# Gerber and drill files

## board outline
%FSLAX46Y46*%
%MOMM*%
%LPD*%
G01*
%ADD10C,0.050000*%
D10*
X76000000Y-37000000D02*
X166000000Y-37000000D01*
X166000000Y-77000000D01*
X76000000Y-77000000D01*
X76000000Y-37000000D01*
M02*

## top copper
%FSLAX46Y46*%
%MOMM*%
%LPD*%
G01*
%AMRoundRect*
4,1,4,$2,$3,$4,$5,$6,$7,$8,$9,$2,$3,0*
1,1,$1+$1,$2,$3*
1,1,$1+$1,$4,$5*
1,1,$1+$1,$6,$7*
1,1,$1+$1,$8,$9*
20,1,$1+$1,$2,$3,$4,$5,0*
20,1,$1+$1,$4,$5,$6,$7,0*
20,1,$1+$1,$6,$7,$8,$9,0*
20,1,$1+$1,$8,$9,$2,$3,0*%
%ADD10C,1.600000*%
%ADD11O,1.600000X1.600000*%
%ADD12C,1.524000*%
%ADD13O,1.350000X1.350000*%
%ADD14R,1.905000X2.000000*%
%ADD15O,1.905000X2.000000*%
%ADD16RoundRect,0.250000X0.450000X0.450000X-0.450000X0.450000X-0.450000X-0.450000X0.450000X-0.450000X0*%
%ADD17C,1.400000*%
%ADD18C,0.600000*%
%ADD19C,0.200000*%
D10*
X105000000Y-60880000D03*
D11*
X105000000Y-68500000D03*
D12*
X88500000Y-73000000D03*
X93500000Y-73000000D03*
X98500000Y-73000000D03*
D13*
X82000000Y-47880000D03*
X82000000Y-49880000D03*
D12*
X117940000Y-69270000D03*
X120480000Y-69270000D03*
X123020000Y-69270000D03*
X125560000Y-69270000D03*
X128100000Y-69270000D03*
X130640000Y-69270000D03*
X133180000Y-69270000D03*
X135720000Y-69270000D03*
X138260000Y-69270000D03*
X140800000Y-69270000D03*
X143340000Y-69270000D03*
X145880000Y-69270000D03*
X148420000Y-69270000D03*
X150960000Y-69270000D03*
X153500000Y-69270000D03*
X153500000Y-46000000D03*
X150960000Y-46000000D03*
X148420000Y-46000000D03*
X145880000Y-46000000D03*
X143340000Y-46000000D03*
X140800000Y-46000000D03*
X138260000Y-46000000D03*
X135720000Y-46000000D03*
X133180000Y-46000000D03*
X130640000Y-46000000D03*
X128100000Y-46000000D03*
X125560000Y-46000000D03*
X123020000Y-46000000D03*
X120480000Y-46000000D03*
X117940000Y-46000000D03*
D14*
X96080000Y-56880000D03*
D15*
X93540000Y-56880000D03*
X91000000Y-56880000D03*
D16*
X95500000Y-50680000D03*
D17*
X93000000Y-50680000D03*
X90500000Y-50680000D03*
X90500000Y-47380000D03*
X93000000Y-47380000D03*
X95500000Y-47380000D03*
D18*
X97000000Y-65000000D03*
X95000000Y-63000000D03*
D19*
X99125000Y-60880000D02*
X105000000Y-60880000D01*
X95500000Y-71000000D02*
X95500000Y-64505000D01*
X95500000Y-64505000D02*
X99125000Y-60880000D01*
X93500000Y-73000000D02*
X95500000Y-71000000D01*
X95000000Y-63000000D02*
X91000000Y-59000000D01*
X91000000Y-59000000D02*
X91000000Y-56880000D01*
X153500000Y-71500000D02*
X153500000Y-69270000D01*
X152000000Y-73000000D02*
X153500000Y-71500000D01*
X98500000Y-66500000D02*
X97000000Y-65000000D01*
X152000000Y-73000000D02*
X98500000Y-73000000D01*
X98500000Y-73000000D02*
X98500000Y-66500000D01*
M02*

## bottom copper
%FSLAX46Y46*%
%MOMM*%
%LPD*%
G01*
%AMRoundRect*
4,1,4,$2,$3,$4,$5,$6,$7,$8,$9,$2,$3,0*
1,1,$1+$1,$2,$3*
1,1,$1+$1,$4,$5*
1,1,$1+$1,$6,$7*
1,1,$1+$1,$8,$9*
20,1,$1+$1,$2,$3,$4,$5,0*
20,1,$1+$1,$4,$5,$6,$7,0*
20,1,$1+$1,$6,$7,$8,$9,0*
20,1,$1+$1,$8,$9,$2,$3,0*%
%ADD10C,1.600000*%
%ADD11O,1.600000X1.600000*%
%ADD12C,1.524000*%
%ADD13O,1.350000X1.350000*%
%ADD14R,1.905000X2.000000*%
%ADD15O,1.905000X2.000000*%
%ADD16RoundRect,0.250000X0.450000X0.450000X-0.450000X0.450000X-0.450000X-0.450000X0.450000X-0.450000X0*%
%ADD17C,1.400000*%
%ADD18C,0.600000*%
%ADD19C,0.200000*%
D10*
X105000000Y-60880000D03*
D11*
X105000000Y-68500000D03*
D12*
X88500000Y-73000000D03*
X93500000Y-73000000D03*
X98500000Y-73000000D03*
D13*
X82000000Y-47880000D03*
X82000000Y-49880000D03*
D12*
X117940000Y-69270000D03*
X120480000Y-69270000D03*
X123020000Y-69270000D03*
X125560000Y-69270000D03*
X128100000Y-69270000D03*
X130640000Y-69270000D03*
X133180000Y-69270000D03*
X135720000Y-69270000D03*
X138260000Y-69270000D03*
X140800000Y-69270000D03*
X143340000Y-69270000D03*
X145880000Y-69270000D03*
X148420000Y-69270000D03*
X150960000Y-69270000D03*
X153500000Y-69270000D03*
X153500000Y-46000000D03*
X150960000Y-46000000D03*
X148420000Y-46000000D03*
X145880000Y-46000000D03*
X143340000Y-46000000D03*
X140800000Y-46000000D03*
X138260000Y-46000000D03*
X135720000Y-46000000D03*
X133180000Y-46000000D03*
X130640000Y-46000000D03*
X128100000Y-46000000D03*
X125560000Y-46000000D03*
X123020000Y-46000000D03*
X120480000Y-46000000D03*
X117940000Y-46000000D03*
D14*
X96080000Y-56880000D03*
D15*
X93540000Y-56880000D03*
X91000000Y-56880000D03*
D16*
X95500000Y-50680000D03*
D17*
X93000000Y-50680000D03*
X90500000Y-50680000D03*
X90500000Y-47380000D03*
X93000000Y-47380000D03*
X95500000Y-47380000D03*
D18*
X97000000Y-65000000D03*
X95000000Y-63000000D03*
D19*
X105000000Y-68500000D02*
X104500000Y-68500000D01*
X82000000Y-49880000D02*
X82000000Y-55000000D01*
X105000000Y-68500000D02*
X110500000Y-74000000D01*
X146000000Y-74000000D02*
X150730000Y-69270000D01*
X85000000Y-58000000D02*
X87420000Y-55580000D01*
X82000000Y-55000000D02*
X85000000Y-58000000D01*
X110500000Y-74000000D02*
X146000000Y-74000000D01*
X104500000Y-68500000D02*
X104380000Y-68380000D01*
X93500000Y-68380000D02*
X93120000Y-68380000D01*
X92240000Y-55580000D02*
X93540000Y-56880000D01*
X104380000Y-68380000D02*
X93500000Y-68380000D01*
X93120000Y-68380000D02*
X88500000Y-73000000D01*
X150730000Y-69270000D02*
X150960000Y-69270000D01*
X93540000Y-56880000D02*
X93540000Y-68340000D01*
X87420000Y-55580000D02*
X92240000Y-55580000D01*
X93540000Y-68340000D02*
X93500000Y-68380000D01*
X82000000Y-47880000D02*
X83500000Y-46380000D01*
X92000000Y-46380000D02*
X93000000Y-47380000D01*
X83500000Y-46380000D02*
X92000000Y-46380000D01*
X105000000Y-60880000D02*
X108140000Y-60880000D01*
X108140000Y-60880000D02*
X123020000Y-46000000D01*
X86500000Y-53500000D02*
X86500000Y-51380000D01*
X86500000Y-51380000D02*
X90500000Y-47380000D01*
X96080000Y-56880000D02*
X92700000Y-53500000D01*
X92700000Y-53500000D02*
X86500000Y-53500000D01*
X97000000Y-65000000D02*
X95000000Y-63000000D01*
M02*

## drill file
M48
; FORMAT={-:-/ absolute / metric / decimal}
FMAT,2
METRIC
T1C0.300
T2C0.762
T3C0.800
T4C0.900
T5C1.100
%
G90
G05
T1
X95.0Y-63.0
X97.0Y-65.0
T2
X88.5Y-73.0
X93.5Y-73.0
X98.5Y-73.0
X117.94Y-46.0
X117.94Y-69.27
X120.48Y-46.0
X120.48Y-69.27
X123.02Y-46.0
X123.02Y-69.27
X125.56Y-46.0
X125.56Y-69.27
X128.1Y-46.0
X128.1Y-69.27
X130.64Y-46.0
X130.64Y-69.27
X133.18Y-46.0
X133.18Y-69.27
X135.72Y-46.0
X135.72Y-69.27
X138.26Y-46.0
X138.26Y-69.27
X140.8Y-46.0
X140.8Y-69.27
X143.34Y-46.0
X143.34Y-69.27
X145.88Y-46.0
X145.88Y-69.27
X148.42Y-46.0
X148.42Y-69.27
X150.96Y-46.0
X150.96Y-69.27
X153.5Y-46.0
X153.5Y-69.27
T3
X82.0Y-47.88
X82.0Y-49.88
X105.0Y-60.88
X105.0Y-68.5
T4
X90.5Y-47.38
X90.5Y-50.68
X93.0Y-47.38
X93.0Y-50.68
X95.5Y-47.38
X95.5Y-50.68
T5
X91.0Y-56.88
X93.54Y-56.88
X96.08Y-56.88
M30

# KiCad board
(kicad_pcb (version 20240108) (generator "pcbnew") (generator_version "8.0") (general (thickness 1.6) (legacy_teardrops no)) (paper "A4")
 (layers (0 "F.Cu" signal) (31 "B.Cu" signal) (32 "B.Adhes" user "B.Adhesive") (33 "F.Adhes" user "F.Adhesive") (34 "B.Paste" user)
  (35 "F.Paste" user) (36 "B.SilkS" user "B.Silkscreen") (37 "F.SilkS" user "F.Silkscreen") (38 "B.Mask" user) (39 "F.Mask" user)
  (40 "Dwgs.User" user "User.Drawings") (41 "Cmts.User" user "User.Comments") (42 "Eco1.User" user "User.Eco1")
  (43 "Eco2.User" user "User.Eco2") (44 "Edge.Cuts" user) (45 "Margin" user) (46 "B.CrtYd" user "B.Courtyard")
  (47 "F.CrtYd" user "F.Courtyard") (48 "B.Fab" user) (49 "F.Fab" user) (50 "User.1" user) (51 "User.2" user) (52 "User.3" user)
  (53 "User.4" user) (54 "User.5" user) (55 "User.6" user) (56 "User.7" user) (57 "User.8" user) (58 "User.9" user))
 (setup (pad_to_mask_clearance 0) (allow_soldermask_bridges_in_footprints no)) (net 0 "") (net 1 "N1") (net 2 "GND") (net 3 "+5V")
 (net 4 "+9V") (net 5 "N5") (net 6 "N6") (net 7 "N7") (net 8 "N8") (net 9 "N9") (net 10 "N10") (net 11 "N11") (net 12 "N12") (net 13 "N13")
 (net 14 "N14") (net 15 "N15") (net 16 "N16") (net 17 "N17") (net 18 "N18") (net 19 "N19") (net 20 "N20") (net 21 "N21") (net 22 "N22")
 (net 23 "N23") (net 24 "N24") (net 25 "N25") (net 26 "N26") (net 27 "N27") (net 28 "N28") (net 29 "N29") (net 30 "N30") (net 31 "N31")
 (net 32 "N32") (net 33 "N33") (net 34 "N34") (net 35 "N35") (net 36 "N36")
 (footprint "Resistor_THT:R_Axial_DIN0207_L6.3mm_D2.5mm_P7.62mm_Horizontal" (layer "F.Cu") (at 105 60.88 -90)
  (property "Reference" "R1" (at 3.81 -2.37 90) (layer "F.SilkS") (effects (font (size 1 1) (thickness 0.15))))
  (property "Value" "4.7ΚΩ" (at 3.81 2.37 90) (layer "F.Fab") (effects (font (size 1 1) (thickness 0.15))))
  (pad "1" thru_hole circle (at 0 0 270) (size 1.6 1.6) (drill 0.8) (layers "*.Cu" "*.Mask") (remove_unused_layers no) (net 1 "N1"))
  (pad "2" thru_hole oval (at 7.62 0 270) (size 1.6 1.6) (drill 0.8) (layers "*.Cu" "*.Mask") (remove_unused_layers no) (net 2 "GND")))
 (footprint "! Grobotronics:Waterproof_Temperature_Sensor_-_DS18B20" (layer "F.Cu") (at 93 66.5)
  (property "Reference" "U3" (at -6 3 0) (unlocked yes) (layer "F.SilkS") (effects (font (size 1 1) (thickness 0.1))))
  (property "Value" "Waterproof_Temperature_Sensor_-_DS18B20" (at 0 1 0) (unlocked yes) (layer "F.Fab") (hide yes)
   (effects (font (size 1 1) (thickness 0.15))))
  (pad "1" thru_hole circle (at -4.5 6.5) (size 1.524 1.524) (drill 0.762) (layers "*.Cu" "*.Mask") (remove_unused_layers no) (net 2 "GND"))
  (pad "2" thru_hole circle (at 0.5 6.5) (size 1.524 1.524) (drill 0.762) (layers "*.Cu" "*.Mask") (remove_unused_layers no) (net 1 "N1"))
  (pad "3" thru_hole circle (at 5.5 6.5) (size 1.524 1.524) (drill 0.762) (layers "*.Cu" "*.Mask") (remove_unused_layers no) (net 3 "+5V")))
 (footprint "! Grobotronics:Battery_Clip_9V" (layer "F.Cu") (at 82 48.38)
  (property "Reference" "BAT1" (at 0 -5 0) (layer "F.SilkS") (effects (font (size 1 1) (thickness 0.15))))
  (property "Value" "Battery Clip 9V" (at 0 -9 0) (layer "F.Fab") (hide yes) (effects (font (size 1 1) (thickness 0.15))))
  (pad "+" thru_hole oval (at 0 -0.5) (size 1.35 1.35) (drill 0.8) (layers "*.Cu" "*.Mask") (remove_unused_layers no) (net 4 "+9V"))
  (pad "-" thru_hole oval (at 0 1.5) (size 1.35 1.35) (drill 0.8) (layers "*.Cu" "*.Mask") (remove_unused_layers no) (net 2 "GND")))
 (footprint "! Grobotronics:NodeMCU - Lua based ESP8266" (layer "F.Cu") (at 135.72 57.77 90)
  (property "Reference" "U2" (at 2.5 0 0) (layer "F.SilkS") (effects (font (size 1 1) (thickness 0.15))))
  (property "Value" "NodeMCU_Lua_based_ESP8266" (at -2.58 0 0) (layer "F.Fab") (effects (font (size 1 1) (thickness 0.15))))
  (pad "1" thru_hole circle (at -11.5 -17.78 90) (size 1.524 1.524) (drill 0.762) (layers "*.Cu" "*.Mask") (remove_unused_layers no)
   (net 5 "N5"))
  (pad "2" thru_hole circle (at -11.5 -15.24 90) (size 1.524 1.524) (drill 0.762) (layers "*.Cu" "*.Mask") (remove_unused_layers no)
   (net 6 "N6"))
  (pad "3" thru_hole circle (at -11.5 -12.7 90) (size 1.524 1.524) (drill 0.762) (layers "*.Cu" "*.Mask") (remove_unused_layers no)
   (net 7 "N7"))
  (pad "4" thru_hole circle (at -11.5 -10.16 90) (size 1.524 1.524) (drill 0.762) (layers "*.Cu" "*.Mask") (remove_unused_layers no)
   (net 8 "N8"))
  (pad "5" thru_hole circle (at -11.5 -7.62 90) (size 1.524 1.524) (drill 0.762) (layers "*.Cu" "*.Mask") (remove_unused_layers no)
   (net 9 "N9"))
  (pad "6" thru_hole circle (at -11.5 -5.08 90) (size 1.524 1.524) (drill 0.762) (layers "*.Cu" "*.Mask") (remove_unused_layers no)
   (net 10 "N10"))
  (pad "7" thru_hole circle (at -11.5 -2.54 90) (size 1.524 1.524) (drill 0.762) (layers "*.Cu" "*.Mask") (remove_unused_layers no)
   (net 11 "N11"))
  (pad "8" thru_hole circle (at -11.5 0 90) (size 1.524 1.524) (drill 0.762) (layers "*.Cu" "*.Mask") (remove_unused_layers no)
   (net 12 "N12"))
  (pad "9" thru_hole circle (at -11.5 2.54 90) (size 1.524 1.524) (drill 0.762) (layers "*.Cu" "*.Mask") (remove_unused_layers no)
   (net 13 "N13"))
  (pad "10" thru_hole circle (at -11.5 5.08 90) (size 1.524 1.524) (drill 0.762) (layers "*.Cu" "*.Mask") (remove_unused_layers no)
   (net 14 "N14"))
  (pad "11" thru_hole circle (at -11.5 7.62 90) (size 1.524 1.524) (drill 0.762) (layers "*.Cu" "*.Mask") (remove_unused_layers no)
   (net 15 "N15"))
  (pad "12" thru_hole circle (at -11.5 10.16 90) (size 1.524 1.524) (drill 0.762) (layers "*.Cu" "*.Mask") (remove_unused_layers no)
   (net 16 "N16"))
  (pad "13" thru_hole circle (at -11.5 12.7 90) (size 1.524 1.524) (drill 0.762) (layers "*.Cu" "*.Mask") (remove_unused_layers no)
   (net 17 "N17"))
  (pad "14" thru_hole circle (at -11.5 15.24 90) (size 1.524 1.524) (drill 0.762) (layers "*.Cu" "*.Mask") (remove_unused_layers no)
   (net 2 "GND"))
  (pad "15" thru_hole circle (at -11.5 17.78 90) (size 1.524 1.524) (drill 0.762) (layers "*.Cu" "*.Mask") (remove_unused_layers no)
   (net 3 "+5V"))
  (pad "16" thru_hole circle (at 11.77 17.78 90) (size 1.524 1.524) (drill 0.762) (layers "*.Cu" "*.Mask") (remove_unused_layers no)
   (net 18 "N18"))
  (pad "17" thru_hole circle (at 11.77 15.24 90) (size 1.524 1.524) (drill 0.762) (layers "*.Cu" "*.Mask") (remove_unused_layers no)
   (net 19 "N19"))
  (pad "18" thru_hole circle (at 11.77 12.7 90) (size 1.524 1.524) (drill 0.762) (layers "*.Cu" "*.Mask") (remove_unused_layers no)
   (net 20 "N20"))
  (pad "19" thru_hole circle (at 11.77 10.16 90) (size 1.524 1.524) (drill 0.762) (layers "*.Cu" "*.Mask") (remove_unused_layers no)
   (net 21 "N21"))
  (pad "20" thru_hole circle (at 11.77 7.62 90) (size 1.524 1.524) (drill 0.762) (layers "*.Cu" "*.Mask") (remove_unused_layers no)
   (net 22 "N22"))
  (pad "21" thru_hole circle (at 11.77 5.08 90) (size 1.524 1.524) (drill 0.762) (layers "*.Cu" "*.Mask") (remove_unused_layers no)
   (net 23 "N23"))
  (pad "22" thru_hole circle (at 11.77 2.54 90) (size 1.524 1.524) (drill 0.762) (layers "*.Cu" "*.Mask") (remove_unused_layers no)
   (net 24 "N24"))
  (pad "23" thru_hole circle (at 11.77 0 90) (size 1.524 1.524) (drill 0.762) (layers "*.Cu" "*.Mask") (remove_unused_layers no)
   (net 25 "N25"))
  (pad "24" thru_hole circle (at 11.77 -2.54 90) (size 1.524 1.524) (drill 0.762) (layers "*.Cu" "*.Mask") (remove_unused_layers no)
   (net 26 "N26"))
  (pad "25" thru_hole circle (at 11.77 -5.08 90) (size 1.524 1.524) (drill 0.762) (layers "*.Cu" "*.Mask") (remove_unused_layers no)
   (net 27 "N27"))
  (pad "26" thru_hole circle (at 11.77 -7.62 90) (size 1.524 1.524) (drill 0.762) (layers "*.Cu" "*.Mask") (remove_unused_layers no)
   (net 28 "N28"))
  (pad "27" thru_hole circle (at 11.77 -10.16 90) (size 1.524 1.524) (drill 0.762) (layers "*.Cu" "*.Mask") (remove_unused_layers no)
   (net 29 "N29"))
  (pad "28" thru_hole circle (at 11.77 -12.7 90) (size 1.524 1.524) (drill 0.762) (layers "*.Cu" "*.Mask") (remove_unused_layers no)
   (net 1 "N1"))
  (pad "29" thru_hole circle (at 11.77 -15.24 90) (size 1.524 1.524) (drill 0.762) (layers "*.Cu" "*.Mask") (remove_unused_layers no)
   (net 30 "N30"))
  (pad "30" thru_hole circle (at 11.77 -17.78 90) (size 1.524 1.524) (drill 0.762) (layers "*.Cu" "*.Mask") (remove_unused_layers no)
   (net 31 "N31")))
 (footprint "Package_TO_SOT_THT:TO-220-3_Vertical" (layer "F.Cu") (at 96.08 56.88 180)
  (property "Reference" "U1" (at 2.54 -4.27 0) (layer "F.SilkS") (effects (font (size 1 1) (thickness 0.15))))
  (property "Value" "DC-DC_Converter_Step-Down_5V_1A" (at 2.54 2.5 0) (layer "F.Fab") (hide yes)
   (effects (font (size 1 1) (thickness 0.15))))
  (pad "1" thru_hole rect (at 0 0 180) (size 1.905 2) (drill 1.1) (layers "*.Cu" "*.Mask") (remove_unused_layers no) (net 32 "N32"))
  (pad "2" thru_hole oval (at 2.54 0 180) (size 1.905 2) (drill 1.1) (layers "*.Cu" "*.Mask") (remove_unused_layers no) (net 2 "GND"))
  (pad "3" thru_hole oval (at 5.08 0 180) (size 1.905 2) (drill 1.1) (layers "*.Cu" "*.Mask") (remove_unused_layers no) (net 3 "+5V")))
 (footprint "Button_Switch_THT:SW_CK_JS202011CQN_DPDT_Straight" (layer "F.Cu") (at 95.5 50.68 180)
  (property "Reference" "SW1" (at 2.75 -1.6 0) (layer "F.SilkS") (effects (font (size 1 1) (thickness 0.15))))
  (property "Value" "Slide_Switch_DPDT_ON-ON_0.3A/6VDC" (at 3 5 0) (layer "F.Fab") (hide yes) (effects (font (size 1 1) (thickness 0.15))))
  (pad "1" thru_hole roundrect (at 0 0 180) (size 1.4 1.4) (drill 0.9) (layers "*.Cu" "*.Mask") (remove_unused_layers no)
   (roundrect_rratio 0.1785714286) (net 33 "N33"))
  (pad "2" thru_hole circle (at 2.5 0 180) (size 1.4 1.4) (drill 0.9) (layers "*.Cu" "*.Mask") (remove_unused_layers no) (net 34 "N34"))
  (pad "3" thru_hole circle (at 5 0 180) (size 1.4 1.4) (drill 0.9) (layers "*.Cu" "*.Mask") (remove_unused_layers no) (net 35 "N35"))
  (pad "4" thru_hole circle (at 5 3.3 180) (size 1.4 1.4) (drill 0.9) (layers "*.Cu" "*.Mask") (remove_unused_layers no) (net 32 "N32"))
  (pad "5" thru_hole circle (at 2.5 3.3 180) (size 1.4 1.4) (drill 0.9) (layers "*.Cu" "*.Mask") (remove_unused_layers no) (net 4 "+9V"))
  (pad "6" thru_hole circle (at 0 3.3 180) (size 1.4 1.4) (drill 0.9) (layers "*.Cu" "*.Mask") (remove_unused_layers no) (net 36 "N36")))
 (gr_rect (start 76 37) (end 166 77) (stroke (width 0.05) (type default)) (fill none) (layer "Edge.Cuts"))
 (segment (start 105 68.5) (end 104.5 68.5) (width 0.2) (layer "B.Cu") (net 2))
 (segment (start 82 49.88) (end 82 55) (width 0.2) (layer "B.Cu") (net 2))
 (segment (start 105 68.5) (end 110.5 74) (width 0.2) (layer "B.Cu") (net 2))
 (segment (start 146 74) (end 150.73 69.27) (width 0.2) (layer "B.Cu") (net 2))
 (segment (start 85 58) (end 87.42 55.58) (width 0.2) (layer "B.Cu") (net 2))
 (segment (start 82 55) (end 85 58) (width 0.2) (layer "B.Cu") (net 2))
 (segment (start 110.5 74) (end 146 74) (width 0.2) (layer "B.Cu") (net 2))
 (segment (start 104.5 68.5) (end 104.38 68.38) (width 0.2) (layer "B.Cu") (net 2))
 (segment (start 93.5 68.38) (end 93.12 68.38) (width 0.2) (layer "B.Cu") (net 2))
 (segment (start 92.24 55.58) (end 93.54 56.88) (width 0.2) (layer "B.Cu") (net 2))
 (segment (start 104.38 68.38) (end 93.5 68.38) (width 0.2) (layer "B.Cu") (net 2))
 (segment (start 93.12 68.38) (end 88.5 73) (width 0.2) (layer "B.Cu") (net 2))
 (segment (start 150.73 69.27) (end 150.96 69.27) (width 0.2) (layer "B.Cu") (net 2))
 (segment (start 93.54 56.88) (end 93.54 68.34) (width 0.2) (layer "B.Cu") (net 2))
 (segment (start 87.42 55.58) (end 92.24 55.58) (width 0.2) (layer "B.Cu") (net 2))
 (segment (start 93.54 68.34) (end 93.5 68.38) (width 0.2) (layer "B.Cu") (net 2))
 (segment (start 82 47.88) (end 83.5 46.38) (width 0.2) (layer "B.Cu") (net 4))
 (segment (start 92 46.38) (end 93 47.38) (width 0.2) (layer "B.Cu") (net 4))
 (segment (start 83.5 46.38) (end 92 46.38) (width 0.2) (layer "B.Cu") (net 4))
 (segment (start 99.125 60.88) (end 105 60.88) (width 0.2) (layer "F.Cu") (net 1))
 (segment (start 95.5 71) (end 95.5 64.505) (width 0.2) (layer "F.Cu") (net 1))
 (segment (start 95.5 64.505) (end 99.125 60.88) (width 0.2) (layer "F.Cu") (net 1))
 (segment (start 93.5 73) (end 95.5 71) (width 0.2) (layer "F.Cu") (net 1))
 (segment (start 105 60.88) (end 108.14 60.88) (width 0.2) (layer "B.Cu") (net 1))
 (segment (start 108.14 60.88) (end 123.02 46) (width 0.2) (layer "B.Cu") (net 1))
 (segment (start 86.5 53.5) (end 86.5 51.38) (width 0.2) (layer "B.Cu") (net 32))
 (segment (start 86.5 51.38) (end 90.5 47.38) (width 0.2) (layer "B.Cu") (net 32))
 (segment (start 96.08 56.88) (end 92.7 53.5) (width 0.2) (layer "B.Cu") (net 32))
 (segment (start 92.7 53.5) (end 86.5 53.5) (width 0.2) (layer "B.Cu") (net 32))
 (segment (start 95 63) (end 91 59) (width 0.2) (layer "F.Cu") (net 3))
 (segment (start 91 59) (end 91 56.88) (width 0.2) (layer "F.Cu") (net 3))
 (segment (start 153.5 71.5) (end 153.5 69.27) (width 0.2) (layer "F.Cu") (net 3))
 (segment (start 152 73) (end 153.5 71.5) (width 0.2) (layer "F.Cu") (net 3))
 (segment (start 98.5 66.5) (end 97 65) (width 0.2) (layer "F.Cu") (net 3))
 (segment (start 152 73) (end 98.5 73) (width 0.2) (layer "F.Cu") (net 3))
 (segment (start 98.5 73) (end 98.5 66.5) (width 0.2) (layer "F.Cu") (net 3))
 (via (at 97 65) (size 0.6) (drill 0.3) (layers "F.Cu" "B.Cu") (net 3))
 (via (at 95 63) (size 0.6) (drill 0.3) (layers "F.Cu" "B.Cu") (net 3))
 (segment (start 97 65) (end 95 63) (width 0.2) (layer "B.Cu") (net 3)))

